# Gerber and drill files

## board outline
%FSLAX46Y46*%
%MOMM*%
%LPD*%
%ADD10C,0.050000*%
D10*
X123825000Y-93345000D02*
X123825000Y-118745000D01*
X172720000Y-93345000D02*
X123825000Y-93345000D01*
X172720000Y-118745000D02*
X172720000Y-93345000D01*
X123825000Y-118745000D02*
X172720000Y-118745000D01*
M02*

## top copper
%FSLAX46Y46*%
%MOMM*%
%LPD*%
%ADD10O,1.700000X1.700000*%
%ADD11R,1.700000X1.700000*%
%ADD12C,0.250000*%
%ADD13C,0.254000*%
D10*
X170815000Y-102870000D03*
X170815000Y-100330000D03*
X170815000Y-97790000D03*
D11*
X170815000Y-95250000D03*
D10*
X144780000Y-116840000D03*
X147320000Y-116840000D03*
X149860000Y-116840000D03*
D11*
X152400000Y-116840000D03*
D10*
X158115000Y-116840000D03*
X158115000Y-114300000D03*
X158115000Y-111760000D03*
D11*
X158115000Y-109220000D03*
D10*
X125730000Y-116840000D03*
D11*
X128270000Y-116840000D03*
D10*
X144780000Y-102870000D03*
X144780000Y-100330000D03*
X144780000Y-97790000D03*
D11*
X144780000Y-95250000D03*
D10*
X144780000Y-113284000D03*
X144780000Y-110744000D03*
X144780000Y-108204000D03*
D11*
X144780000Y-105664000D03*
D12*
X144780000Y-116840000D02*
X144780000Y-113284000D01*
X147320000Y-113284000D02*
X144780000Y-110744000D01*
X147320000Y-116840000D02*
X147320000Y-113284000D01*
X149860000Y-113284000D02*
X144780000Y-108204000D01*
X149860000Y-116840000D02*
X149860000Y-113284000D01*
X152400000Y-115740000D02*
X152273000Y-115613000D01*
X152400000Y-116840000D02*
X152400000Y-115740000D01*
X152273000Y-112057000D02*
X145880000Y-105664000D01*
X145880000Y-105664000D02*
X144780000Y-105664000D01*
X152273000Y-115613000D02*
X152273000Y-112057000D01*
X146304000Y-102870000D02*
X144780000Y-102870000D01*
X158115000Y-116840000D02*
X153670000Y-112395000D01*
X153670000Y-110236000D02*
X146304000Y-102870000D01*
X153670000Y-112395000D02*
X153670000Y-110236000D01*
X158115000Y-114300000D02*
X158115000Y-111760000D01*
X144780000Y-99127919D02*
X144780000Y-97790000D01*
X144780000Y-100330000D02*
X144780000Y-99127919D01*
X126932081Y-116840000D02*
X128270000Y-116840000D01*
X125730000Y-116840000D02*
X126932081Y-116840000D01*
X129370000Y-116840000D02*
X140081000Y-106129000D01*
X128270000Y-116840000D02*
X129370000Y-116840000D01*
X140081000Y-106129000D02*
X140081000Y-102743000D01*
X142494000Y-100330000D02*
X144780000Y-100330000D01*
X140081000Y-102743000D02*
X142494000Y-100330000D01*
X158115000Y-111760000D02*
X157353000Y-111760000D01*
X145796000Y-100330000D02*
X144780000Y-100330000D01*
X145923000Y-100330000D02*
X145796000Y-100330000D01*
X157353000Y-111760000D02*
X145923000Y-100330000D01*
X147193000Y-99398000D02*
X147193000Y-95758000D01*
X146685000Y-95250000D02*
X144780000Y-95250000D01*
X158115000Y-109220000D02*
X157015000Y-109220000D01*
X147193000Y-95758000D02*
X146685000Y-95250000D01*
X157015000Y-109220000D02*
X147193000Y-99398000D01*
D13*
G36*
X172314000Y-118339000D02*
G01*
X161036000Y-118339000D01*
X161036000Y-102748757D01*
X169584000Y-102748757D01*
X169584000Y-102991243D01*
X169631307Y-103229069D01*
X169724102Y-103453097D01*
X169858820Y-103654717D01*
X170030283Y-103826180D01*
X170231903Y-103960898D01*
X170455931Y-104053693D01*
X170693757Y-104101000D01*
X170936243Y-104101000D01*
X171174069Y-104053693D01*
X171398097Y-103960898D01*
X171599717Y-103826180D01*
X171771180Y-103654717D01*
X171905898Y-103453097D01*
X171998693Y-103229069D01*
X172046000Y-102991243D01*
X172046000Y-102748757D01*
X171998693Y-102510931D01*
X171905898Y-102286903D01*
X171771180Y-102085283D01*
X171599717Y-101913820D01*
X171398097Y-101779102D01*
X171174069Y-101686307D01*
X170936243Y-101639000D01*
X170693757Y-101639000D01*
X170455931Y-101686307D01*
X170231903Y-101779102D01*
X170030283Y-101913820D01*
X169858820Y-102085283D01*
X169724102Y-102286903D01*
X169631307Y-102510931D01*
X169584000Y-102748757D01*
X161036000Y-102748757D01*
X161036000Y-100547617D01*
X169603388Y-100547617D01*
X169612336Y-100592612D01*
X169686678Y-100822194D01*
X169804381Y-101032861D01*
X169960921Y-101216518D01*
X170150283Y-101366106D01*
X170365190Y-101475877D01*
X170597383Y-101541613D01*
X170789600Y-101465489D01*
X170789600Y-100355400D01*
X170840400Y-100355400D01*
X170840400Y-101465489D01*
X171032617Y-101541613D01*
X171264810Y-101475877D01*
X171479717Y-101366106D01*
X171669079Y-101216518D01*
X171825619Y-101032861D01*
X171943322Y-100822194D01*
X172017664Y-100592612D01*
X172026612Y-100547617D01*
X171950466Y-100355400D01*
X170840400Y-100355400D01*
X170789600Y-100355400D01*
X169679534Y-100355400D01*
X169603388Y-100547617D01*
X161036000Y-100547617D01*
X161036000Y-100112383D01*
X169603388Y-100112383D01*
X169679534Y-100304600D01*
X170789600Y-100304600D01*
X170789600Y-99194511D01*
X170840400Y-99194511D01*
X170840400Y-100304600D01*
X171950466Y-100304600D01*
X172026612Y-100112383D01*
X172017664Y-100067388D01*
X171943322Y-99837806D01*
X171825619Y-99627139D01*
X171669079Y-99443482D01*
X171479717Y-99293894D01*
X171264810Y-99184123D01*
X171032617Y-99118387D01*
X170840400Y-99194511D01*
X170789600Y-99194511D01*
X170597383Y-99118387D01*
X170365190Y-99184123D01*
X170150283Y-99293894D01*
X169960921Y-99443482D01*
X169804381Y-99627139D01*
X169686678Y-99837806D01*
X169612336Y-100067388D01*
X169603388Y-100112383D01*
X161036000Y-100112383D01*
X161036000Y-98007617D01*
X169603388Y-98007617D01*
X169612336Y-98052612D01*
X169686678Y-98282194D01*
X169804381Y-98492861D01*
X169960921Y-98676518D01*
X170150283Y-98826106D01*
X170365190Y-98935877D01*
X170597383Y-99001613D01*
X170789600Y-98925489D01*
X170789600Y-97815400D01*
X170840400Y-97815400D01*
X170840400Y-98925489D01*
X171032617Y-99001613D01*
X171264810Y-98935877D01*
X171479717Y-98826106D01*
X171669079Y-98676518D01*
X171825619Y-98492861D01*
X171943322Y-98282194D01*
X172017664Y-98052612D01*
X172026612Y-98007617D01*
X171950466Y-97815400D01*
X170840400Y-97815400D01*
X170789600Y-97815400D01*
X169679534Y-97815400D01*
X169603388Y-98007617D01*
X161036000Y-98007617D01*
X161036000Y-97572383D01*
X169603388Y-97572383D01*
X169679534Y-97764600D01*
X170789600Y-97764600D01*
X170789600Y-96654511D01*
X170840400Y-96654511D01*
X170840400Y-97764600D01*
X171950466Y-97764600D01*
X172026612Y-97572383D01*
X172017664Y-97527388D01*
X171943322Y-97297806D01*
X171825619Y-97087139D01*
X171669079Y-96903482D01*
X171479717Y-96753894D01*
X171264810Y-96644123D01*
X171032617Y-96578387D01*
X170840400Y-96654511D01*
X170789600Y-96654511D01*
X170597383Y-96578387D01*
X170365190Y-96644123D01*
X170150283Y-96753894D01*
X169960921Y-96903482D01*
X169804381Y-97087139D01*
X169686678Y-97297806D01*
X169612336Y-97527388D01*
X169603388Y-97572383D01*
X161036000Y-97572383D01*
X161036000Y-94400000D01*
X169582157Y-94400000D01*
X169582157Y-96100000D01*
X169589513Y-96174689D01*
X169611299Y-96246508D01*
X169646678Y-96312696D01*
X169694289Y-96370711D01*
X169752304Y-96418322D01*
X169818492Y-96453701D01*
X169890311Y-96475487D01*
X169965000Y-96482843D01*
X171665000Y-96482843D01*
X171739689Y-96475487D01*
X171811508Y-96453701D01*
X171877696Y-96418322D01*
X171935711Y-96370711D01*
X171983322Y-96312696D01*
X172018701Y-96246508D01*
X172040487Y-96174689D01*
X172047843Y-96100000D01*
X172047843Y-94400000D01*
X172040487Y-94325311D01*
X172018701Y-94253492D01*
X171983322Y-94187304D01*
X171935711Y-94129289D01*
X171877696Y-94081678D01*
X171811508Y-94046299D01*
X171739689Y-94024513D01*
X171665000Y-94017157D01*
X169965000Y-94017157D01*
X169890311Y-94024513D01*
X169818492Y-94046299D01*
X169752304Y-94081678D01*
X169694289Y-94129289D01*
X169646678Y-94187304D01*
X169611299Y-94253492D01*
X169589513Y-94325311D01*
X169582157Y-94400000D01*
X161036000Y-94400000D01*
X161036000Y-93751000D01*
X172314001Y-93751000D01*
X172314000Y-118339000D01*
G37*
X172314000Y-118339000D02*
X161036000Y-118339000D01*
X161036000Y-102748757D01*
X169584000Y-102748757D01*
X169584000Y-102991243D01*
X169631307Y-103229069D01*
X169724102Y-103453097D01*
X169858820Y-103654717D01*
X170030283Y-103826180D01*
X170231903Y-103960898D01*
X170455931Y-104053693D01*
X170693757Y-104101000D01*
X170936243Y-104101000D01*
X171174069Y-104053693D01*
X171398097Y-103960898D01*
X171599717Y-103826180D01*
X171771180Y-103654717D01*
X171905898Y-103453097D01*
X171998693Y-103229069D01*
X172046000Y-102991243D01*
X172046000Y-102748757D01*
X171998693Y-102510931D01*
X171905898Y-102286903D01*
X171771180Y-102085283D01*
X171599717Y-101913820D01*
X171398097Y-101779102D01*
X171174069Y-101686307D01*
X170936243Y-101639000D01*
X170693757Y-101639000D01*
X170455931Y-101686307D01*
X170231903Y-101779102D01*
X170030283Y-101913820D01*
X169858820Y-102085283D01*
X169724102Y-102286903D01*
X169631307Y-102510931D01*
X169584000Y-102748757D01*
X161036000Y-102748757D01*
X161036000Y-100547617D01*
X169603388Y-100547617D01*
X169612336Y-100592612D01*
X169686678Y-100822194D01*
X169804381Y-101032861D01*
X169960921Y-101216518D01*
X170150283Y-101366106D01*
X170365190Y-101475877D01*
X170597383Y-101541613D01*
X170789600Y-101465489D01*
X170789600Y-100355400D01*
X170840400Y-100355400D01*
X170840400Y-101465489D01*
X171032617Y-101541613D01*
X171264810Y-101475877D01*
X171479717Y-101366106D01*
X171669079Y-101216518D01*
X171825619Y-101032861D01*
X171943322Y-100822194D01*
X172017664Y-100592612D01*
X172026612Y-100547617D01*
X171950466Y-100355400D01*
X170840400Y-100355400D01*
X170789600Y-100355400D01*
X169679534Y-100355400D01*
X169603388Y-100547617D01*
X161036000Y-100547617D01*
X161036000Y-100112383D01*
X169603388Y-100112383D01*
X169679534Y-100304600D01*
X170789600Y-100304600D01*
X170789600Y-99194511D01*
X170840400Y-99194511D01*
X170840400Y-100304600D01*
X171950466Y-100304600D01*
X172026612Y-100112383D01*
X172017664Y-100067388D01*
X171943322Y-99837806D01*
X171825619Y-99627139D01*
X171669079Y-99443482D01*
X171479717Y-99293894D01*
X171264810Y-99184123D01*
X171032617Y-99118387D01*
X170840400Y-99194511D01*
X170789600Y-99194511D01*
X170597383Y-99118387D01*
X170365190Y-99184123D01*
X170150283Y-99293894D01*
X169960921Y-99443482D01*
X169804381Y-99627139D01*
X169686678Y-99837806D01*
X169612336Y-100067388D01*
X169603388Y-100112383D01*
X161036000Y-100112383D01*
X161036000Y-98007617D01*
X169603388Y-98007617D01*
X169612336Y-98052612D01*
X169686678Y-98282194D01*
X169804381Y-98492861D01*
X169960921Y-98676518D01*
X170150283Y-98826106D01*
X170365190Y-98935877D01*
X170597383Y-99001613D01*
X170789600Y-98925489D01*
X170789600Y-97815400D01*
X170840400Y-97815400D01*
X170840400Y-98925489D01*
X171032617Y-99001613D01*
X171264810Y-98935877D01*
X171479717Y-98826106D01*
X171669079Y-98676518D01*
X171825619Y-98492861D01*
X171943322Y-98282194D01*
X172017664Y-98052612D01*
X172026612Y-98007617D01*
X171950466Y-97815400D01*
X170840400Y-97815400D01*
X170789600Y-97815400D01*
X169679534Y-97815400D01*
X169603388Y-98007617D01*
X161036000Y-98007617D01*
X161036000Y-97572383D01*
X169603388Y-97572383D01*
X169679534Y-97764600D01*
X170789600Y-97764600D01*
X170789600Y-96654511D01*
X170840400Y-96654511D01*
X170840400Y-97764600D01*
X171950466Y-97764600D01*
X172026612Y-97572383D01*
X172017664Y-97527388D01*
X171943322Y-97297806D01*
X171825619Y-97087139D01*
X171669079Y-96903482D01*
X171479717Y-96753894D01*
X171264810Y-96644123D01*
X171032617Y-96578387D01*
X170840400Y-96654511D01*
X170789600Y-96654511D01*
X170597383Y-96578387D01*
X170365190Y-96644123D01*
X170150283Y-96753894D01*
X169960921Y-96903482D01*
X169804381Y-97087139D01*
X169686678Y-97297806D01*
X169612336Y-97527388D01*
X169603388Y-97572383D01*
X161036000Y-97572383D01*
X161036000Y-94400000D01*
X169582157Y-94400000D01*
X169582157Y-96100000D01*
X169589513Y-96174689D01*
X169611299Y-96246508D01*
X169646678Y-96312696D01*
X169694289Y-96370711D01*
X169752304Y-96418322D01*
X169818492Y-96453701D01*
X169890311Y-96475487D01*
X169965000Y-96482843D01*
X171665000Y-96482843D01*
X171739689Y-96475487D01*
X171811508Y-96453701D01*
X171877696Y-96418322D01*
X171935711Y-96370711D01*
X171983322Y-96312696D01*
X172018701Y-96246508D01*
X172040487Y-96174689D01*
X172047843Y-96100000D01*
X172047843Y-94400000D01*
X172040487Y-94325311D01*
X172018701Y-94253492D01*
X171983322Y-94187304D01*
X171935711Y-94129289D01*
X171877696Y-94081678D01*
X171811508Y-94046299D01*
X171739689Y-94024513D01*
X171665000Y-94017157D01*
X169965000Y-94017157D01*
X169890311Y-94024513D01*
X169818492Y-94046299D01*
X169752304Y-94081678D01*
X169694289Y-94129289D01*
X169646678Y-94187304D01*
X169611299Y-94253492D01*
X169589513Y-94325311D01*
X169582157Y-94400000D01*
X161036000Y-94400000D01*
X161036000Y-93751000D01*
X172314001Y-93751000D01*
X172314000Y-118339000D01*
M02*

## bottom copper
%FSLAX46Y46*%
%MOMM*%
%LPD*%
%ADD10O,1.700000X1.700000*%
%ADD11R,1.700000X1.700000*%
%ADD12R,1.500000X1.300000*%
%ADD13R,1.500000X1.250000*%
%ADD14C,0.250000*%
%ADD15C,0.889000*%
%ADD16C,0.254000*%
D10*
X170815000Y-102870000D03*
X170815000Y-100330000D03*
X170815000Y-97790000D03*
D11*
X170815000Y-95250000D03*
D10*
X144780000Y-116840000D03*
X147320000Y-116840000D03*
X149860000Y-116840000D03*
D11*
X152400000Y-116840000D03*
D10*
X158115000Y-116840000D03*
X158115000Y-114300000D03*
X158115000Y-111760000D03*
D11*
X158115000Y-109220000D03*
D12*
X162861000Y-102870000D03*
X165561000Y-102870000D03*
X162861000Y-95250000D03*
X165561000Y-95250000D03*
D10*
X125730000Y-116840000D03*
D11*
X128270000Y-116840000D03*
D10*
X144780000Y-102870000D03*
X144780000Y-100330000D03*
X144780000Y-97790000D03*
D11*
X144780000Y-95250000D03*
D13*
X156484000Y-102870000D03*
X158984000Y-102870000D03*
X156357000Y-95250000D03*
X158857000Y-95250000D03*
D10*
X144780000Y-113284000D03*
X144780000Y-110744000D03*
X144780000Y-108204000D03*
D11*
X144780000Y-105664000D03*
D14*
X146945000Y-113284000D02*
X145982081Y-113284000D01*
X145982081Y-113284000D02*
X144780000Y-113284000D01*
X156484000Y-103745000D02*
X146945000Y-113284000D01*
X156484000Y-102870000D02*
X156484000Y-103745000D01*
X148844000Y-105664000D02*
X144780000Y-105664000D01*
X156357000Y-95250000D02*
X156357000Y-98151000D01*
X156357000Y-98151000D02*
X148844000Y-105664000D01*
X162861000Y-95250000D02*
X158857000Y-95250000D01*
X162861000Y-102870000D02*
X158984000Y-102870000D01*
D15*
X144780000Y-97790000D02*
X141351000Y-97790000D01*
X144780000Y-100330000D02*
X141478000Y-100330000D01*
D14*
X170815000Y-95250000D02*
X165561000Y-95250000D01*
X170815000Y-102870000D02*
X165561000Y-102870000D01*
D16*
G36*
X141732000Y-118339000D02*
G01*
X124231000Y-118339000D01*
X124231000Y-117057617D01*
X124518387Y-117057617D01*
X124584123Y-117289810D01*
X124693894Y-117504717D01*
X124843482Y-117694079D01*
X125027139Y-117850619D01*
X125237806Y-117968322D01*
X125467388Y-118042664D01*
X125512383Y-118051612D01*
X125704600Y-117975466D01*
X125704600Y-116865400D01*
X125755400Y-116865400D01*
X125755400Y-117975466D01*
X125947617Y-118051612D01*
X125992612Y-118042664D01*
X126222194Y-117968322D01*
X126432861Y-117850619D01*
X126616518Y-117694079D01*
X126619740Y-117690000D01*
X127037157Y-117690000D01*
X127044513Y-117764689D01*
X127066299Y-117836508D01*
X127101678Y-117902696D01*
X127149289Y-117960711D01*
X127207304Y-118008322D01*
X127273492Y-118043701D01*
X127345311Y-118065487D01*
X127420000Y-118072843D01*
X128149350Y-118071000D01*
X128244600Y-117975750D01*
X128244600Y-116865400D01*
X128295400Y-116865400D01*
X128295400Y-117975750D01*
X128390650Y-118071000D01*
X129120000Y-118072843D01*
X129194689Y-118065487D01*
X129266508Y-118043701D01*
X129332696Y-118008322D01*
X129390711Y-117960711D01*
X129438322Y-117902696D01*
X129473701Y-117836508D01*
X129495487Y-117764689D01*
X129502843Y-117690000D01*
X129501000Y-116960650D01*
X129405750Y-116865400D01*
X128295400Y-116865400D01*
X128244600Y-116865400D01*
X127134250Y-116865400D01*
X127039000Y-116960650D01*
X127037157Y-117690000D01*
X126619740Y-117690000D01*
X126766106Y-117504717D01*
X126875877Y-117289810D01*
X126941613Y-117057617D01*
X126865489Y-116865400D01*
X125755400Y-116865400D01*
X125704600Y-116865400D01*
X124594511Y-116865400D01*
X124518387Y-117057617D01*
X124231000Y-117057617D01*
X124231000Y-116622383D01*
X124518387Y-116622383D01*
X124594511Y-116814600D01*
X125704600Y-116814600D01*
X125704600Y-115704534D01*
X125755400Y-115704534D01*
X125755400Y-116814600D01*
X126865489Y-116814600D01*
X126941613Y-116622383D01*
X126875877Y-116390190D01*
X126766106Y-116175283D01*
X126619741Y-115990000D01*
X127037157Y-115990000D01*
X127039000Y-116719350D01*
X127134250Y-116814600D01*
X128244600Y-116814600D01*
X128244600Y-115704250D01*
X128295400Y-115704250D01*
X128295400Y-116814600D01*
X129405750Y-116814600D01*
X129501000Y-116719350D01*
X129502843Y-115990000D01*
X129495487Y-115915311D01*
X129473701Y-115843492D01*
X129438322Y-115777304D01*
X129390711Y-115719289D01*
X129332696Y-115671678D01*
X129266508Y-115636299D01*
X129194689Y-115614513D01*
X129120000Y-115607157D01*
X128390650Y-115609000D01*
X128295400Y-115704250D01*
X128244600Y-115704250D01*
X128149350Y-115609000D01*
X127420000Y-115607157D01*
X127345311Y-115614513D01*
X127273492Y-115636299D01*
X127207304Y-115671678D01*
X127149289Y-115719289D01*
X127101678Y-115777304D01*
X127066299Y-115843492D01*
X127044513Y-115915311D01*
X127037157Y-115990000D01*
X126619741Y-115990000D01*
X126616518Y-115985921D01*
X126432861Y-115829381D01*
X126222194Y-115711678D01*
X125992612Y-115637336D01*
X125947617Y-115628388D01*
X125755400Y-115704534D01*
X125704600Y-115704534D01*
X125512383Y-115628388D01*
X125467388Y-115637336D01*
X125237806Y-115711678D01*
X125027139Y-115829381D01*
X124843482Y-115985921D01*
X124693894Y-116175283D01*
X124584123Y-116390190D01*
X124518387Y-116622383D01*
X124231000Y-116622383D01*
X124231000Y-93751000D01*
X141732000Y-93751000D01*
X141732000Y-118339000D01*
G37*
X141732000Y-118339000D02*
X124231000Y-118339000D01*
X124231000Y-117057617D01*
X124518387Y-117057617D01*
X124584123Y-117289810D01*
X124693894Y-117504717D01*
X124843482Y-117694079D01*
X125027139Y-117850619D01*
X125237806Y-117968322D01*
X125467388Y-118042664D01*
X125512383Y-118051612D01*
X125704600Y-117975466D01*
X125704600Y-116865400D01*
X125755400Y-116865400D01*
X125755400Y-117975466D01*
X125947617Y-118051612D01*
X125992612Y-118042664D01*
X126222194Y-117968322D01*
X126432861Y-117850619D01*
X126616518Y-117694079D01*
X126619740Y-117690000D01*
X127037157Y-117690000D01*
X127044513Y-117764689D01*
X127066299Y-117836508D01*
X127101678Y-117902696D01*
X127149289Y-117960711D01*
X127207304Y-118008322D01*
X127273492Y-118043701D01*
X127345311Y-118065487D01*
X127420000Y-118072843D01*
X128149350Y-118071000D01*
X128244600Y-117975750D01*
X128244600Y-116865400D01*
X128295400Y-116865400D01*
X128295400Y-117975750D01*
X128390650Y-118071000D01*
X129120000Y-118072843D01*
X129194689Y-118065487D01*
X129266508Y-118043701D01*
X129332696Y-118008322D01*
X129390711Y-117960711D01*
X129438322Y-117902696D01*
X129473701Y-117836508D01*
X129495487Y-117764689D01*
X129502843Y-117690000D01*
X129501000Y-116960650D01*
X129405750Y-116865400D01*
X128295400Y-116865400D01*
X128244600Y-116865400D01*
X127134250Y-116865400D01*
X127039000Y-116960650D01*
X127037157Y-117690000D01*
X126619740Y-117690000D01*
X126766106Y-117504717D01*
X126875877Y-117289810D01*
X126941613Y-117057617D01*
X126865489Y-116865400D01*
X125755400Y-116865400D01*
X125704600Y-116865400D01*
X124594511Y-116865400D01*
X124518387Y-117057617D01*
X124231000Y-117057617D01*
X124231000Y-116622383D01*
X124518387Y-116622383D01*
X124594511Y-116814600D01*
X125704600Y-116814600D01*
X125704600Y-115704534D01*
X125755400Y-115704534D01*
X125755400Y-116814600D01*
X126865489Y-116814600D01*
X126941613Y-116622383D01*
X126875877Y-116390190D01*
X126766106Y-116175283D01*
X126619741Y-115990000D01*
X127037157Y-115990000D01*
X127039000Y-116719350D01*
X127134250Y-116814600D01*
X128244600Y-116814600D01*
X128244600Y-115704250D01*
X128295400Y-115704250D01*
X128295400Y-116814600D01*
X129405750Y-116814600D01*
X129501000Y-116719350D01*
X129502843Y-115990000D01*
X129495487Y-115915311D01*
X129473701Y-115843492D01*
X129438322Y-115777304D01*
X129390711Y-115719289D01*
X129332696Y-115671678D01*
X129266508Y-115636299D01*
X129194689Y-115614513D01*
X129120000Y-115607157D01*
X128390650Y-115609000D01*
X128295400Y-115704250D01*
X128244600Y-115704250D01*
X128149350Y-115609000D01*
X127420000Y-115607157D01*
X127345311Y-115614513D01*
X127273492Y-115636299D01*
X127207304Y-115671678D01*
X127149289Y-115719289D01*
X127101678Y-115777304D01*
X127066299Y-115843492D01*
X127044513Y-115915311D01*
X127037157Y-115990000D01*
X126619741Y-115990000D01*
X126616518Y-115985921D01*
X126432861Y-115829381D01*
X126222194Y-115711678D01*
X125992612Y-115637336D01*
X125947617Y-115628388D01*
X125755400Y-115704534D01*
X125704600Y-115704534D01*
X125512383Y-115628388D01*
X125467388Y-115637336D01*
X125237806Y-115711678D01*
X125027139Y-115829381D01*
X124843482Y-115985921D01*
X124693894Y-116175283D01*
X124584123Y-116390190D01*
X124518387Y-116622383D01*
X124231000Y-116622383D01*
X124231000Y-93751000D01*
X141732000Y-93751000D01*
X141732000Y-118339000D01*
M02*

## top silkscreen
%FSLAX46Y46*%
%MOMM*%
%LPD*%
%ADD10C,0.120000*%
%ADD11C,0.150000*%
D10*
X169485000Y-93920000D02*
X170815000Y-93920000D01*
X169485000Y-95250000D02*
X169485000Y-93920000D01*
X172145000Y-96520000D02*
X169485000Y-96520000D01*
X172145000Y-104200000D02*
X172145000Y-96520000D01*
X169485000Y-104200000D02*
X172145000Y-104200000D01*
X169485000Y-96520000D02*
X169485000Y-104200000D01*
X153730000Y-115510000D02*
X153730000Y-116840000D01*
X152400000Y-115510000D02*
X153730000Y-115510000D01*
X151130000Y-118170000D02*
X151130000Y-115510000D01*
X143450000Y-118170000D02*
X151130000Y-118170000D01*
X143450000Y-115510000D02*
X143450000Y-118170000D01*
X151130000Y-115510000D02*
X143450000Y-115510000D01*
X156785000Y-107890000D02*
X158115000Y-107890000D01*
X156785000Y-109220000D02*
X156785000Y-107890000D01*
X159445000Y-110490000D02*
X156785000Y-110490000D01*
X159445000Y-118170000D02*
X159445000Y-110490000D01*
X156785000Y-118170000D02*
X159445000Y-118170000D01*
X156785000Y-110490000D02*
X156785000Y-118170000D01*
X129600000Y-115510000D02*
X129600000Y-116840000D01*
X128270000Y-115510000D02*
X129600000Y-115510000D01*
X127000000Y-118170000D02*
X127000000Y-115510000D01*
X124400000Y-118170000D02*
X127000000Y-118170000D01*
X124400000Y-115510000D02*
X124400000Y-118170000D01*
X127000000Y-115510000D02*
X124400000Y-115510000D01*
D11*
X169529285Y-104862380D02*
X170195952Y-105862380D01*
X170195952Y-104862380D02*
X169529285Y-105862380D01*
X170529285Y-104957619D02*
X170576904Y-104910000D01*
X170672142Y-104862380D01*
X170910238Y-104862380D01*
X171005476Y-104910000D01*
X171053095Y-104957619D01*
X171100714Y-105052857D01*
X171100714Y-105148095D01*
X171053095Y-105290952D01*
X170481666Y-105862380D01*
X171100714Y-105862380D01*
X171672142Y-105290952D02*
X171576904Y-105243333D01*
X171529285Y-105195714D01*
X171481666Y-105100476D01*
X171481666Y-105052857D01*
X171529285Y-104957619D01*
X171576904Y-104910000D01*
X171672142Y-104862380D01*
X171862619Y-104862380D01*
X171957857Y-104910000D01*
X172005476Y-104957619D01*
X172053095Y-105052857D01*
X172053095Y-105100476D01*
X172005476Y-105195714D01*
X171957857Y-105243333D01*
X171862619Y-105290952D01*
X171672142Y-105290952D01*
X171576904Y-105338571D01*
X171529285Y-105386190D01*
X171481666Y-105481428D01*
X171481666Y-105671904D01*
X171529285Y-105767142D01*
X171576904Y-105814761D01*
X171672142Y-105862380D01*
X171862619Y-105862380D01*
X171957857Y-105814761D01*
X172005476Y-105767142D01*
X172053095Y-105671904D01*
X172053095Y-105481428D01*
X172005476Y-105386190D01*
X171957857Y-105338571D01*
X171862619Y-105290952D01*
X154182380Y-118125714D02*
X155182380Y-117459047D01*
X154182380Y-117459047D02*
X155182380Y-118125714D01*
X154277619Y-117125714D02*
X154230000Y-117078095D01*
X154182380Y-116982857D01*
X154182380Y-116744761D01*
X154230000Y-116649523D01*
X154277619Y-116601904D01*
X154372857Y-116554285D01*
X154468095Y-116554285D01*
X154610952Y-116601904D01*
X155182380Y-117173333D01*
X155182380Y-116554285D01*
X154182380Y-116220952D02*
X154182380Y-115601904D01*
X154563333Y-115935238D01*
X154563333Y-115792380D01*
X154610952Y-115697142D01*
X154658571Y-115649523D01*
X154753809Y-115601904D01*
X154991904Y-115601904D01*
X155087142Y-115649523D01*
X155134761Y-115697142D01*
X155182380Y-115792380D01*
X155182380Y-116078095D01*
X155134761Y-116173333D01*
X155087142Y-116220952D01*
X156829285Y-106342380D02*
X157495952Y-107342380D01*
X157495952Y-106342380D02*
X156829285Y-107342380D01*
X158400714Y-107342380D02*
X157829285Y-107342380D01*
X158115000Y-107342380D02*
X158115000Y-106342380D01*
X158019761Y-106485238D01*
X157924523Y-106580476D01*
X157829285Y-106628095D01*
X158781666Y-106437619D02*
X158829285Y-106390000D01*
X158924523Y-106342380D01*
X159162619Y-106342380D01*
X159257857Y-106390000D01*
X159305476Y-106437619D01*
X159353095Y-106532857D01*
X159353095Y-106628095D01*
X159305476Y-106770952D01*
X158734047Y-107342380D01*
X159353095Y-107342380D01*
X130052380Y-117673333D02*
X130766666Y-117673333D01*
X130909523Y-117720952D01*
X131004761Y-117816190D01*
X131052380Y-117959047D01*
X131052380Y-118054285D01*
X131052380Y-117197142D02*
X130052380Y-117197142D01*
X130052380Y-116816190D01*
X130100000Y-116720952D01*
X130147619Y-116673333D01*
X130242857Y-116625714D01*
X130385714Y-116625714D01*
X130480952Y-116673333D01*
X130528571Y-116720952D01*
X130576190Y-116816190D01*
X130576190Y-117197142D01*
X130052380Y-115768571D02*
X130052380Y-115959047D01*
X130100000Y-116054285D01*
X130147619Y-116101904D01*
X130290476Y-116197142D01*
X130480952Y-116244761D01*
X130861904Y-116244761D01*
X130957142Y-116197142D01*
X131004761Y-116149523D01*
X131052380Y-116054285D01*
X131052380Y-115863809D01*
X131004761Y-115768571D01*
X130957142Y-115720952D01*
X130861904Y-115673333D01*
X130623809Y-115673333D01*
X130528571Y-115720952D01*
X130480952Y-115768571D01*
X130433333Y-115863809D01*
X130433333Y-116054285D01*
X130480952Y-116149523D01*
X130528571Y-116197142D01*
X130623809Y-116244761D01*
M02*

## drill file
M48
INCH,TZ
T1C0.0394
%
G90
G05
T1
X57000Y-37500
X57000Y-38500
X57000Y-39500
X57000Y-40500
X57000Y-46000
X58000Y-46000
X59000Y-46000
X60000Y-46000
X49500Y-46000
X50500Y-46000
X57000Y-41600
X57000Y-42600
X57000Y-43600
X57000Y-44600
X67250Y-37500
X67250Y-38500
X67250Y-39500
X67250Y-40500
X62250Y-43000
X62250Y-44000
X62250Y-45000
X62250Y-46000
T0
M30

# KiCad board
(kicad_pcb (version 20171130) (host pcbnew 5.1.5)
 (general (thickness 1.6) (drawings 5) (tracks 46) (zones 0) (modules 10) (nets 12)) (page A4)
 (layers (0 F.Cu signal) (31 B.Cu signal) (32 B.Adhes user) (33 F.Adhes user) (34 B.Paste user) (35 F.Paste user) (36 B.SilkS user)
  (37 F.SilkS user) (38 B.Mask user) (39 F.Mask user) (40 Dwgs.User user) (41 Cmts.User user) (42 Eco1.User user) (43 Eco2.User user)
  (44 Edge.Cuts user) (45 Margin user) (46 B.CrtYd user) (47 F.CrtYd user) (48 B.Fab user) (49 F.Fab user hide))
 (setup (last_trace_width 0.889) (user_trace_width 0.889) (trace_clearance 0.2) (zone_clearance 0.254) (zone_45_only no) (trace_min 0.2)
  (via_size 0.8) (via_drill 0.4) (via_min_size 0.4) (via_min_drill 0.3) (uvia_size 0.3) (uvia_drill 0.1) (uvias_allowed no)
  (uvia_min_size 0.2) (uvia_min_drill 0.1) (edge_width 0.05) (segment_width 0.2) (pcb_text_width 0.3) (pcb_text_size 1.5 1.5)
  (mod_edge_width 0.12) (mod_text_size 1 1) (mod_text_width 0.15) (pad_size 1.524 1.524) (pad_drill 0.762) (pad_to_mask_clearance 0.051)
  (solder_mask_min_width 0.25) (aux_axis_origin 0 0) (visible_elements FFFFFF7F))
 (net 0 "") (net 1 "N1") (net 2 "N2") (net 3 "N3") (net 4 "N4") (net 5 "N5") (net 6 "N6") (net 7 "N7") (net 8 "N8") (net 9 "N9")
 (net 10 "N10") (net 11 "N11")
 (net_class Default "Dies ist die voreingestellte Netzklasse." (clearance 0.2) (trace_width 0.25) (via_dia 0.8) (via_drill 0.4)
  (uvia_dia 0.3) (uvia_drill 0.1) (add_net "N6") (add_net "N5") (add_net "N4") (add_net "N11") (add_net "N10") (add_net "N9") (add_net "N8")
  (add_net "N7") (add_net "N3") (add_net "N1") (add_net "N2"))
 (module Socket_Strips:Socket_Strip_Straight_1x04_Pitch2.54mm (layer F.Cu) (at 170.815 95.25)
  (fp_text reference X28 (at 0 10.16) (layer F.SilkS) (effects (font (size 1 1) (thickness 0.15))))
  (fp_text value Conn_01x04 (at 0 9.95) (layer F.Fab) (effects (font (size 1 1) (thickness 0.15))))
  (fp_line (start -1.33 -1.33) (end 0 -1.33) (layer F.SilkS) (width 0.12))
  (fp_line (start -1.33 0) (end -1.33 -1.33) (layer F.SilkS) (width 0.12))
  (fp_line (start 1.33 1.27) (end -1.33 1.27) (layer F.SilkS) (width 0.12))
  (fp_line (start 1.33 8.95) (end 1.33 1.27) (layer F.SilkS) (width 0.12))
  (fp_line (start -1.33 8.95) (end 1.33 8.95) (layer F.SilkS) (width 0.12))
  (fp_line (start -1.33 1.27) (end -1.33 8.95) (layer F.SilkS) (width 0.12))
  (pad 4 thru_hole oval (at 0 7.62) (size 1.7 1.7) (drill 1) (layers *.Cu *.Mask) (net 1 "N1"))
  (pad 3 thru_hole oval (at 0 5.08) (size 1.7 1.7) (drill 1) (layers *.Cu *.Mask) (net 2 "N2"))
  (pad 2 thru_hole oval (at 0 2.54) (size 1.7 1.7) (drill 1) (layers *.Cu *.Mask) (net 2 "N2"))
  (pad 1 thru_hole rect (at 0 0) (size 1.7 1.7) (drill 1) (layers *.Cu *.Mask) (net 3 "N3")))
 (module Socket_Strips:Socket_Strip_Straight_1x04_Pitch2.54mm (layer F.Cu) (at 152.4 116.84 270)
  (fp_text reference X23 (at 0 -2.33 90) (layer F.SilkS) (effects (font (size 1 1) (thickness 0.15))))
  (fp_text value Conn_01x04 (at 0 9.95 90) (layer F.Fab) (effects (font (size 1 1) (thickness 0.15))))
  (fp_line (start -1.33 -1.33) (end 0 -1.33) (layer F.SilkS) (width 0.12))
  (fp_line (start -1.33 0) (end -1.33 -1.33) (layer F.SilkS) (width 0.12))
  (fp_line (start 1.33 1.27) (end -1.33 1.27) (layer F.SilkS) (width 0.12))
  (fp_line (start 1.33 8.95) (end 1.33 1.27) (layer F.SilkS) (width 0.12))
  (fp_line (start -1.33 8.95) (end 1.33 8.95) (layer F.SilkS) (width 0.12))
  (fp_line (start -1.33 1.27) (end -1.33 8.95) (layer F.SilkS) (width 0.12))
  (pad 4 thru_hole oval (at 0 7.62 270) (size 1.7 1.7) (drill 1) (layers *.Cu *.Mask) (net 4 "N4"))
  (pad 3 thru_hole oval (at 0 5.08 270) (size 1.7 1.7) (drill 1) (layers *.Cu *.Mask) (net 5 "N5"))
  (pad 2 thru_hole oval (at 0 2.54 270) (size 1.7 1.7) (drill 1) (layers *.Cu *.Mask) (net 5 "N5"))
  (pad 1 thru_hole rect (at 0 0 270) (size 1.7 1.7) (drill 1) (layers *.Cu *.Mask) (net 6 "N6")))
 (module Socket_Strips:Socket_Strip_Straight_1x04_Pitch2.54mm (layer F.Cu) (at 158.115 109.22)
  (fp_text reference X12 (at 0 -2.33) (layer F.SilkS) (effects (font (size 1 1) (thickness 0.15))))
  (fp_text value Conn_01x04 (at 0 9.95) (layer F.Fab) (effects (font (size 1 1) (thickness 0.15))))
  (fp_line (start -1.33 -1.33) (end 0 -1.33) (layer F.SilkS) (width 0.12))
  (fp_line (start -1.33 0) (end -1.33 -1.33) (layer F.SilkS) (width 0.12))
  (fp_line (start 1.33 1.27) (end -1.33 1.27) (layer F.SilkS) (width 0.12))
  (fp_line (start 1.33 8.95) (end 1.33 1.27) (layer F.SilkS) (width 0.12))
  (fp_line (start -1.33 8.95) (end 1.33 8.95) (layer F.SilkS) (width 0.12))
  (fp_line (start -1.33 1.27) (end -1.33 8.95) (layer F.SilkS) (width 0.12))
  (pad 4 thru_hole oval (at 0 7.62) (size 1.7 1.7) (drill 1) (layers *.Cu *.Mask) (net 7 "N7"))
  (pad 3 thru_hole oval (at 0 5.08) (size 1.7 1.7) (drill 1) (layers *.Cu *.Mask) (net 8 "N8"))
  (pad 2 thru_hole oval (at 0 2.54) (size 1.7 1.7) (drill 1) (layers *.Cu *.Mask) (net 8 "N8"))
  (pad 1 thru_hole rect (at 0 0) (size 1.7 1.7) (drill 1) (layers *.Cu *.Mask) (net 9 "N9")))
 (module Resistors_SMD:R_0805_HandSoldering (layer B.Cu) (at 164.211 102.87 180)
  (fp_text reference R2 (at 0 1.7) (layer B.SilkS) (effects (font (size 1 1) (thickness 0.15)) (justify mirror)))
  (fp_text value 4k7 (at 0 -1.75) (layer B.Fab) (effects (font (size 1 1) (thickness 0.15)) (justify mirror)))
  (pad 2 smd rect (at 1.35 0 180) (size 1.5 1.3) (layers B.Cu B.Paste B.Mask) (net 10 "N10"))
  (pad 1 smd rect (at -1.35 0 180) (size 1.5 1.3) (layers B.Cu B.Paste B.Mask) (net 1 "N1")))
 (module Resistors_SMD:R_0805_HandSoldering (layer B.Cu) (at 164.211 95.25 180)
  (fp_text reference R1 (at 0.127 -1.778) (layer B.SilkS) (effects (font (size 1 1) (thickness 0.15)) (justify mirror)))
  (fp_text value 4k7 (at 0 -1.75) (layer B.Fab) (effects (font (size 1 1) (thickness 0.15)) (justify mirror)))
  (pad 2 smd rect (at 1.35 0 180) (size 1.5 1.3) (layers B.Cu B.Paste B.Mask) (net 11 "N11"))
  (pad 1 smd rect (at -1.35 0 180) (size 1.5 1.3) (layers B.Cu B.Paste B.Mask) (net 3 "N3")))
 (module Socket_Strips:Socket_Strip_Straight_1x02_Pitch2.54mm (layer F.Cu) (at 128.27 116.84 270)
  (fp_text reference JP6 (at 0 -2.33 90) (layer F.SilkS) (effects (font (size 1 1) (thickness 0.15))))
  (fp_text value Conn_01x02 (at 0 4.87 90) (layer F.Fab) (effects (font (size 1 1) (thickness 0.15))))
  (fp_line (start -1.33 -1.33) (end 0 -1.33) (layer F.SilkS) (width 0.12))
  (fp_line (start -1.33 0) (end -1.33 -1.33) (layer F.SilkS) (width 0.12))
  (fp_line (start 1.33 1.27) (end -1.33 1.27) (layer F.SilkS) (width 0.12))
  (fp_line (start 1.33 3.87) (end 1.33 1.27) (layer F.SilkS) (width 0.12))
  (fp_line (start -1.33 3.87) (end 1.33 3.87) (layer F.SilkS) (width 0.12))
  (fp_line (start -1.33 1.27) (end -1.33 3.87) (layer F.SilkS) (width 0.12))
  (pad 2 thru_hole oval (at 0 2.54 270) (size 1.7 1.7) (drill 1) (layers *.Cu *.Mask) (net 8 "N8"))
  (pad 1 thru_hole rect (at 0 0 270) (size 1.7 1.7) (drill 1) (layers *.Cu *.Mask) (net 8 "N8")))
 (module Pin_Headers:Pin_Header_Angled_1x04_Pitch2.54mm (layer B.Cu) (at 144.78 95.25 180)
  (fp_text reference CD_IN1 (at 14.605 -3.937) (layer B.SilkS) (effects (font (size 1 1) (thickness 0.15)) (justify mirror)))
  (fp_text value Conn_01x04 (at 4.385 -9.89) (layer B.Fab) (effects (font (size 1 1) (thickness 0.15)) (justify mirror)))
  (pad 4 thru_hole oval (at 0 -7.62 180) (size 1.7 1.7) (drill 1) (layers *.Cu *.Mask) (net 7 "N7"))
  (pad 3 thru_hole oval (at 0 -5.08 180) (size 1.7 1.7) (drill 1) (layers *.Cu *.Mask) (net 8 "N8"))
  (pad 2 thru_hole oval (at 0 -2.54 180) (size 1.7 1.7) (drill 1) (layers *.Cu *.Mask) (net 8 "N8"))
  (pad 1 thru_hole rect (at 0 0 180) (size 1.7 1.7) (drill 1) (layers *.Cu *.Mask) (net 9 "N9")))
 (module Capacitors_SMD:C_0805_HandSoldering (layer B.Cu) (at 157.734 102.87 180)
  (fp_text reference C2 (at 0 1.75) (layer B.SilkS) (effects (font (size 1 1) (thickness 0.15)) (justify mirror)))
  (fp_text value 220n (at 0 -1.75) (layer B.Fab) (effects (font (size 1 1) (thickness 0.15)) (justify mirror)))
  (pad 2 smd rect (at 1.25 0 180) (size 1.5 1.25) (layers B.Cu B.Paste B.Mask) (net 4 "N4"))
  (pad 1 smd rect (at -1.25 0 180) (size 1.5 1.25) (layers B.Cu B.Paste B.Mask) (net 10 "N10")))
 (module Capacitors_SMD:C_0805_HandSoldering (layer B.Cu) (at 157.607 95.25 180)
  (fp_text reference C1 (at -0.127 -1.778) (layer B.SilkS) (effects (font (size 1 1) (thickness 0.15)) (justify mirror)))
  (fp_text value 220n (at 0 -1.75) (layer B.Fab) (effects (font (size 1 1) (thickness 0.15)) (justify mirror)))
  (pad 2 smd rect (at 1.25 0 180) (size 1.5 1.25) (layers B.Cu B.Paste B.Mask) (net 6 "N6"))
  (pad 1 smd rect (at -1.25 0 180) (size 1.5 1.25) (layers B.Cu B.Paste B.Mask) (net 11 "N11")))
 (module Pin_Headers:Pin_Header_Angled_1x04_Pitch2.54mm (layer B.Cu) (at 144.78 105.664 180)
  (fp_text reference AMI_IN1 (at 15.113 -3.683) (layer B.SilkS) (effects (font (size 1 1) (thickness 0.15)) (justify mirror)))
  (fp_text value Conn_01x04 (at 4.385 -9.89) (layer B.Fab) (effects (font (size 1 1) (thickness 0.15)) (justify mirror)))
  (pad 4 thru_hole oval (at 0 -7.62 180) (size 1.7 1.7) (drill 1) (layers *.Cu *.Mask) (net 4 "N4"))
  (pad 3 thru_hole oval (at 0 -5.08 180) (size 1.7 1.7) (drill 1) (layers *.Cu *.Mask) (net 5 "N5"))
  (pad 2 thru_hole oval (at 0 -2.54 180) (size 1.7 1.7) (drill 1) (layers *.Cu *.Mask) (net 5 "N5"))
  (pad 1 thru_hole rect (at 0 0 180) (size 1.7 1.7) (drill 1) (layers *.Cu *.Mask) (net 6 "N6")))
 (gr_line (start 123.825 93.345) (end 123.825 118.745) (layer Edge.Cuts) (width 0.05))
 (gr_line (start 172.72 93.345) (end 123.825 93.345) (layer Edge.Cuts) (width 0.05))
 (gr_line (start 172.72 118.745) (end 172.72 93.345) (layer Edge.Cuts) (width 0.05))
 (gr_line (start 123.825 118.745) (end 172.72 118.745) (layer Edge.Cuts) (width 0.05))
 (segment (start 144.78 116.84) (end 144.78 113.284) (width 0.25) (layer F.Cu) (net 4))
 (segment (start 146.945 113.284) (end 145.982081 113.284) (width 0.25) (layer B.Cu) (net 4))
 (segment (start 145.982081 113.284) (end 144.78 113.284) (width 0.25) (layer B.Cu) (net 4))
 (segment (start 156.484 103.745) (end 146.945 113.284) (width 0.25) (layer B.Cu) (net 4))
 (segment (start 156.484 102.87) (end 156.484 103.745) (width 0.25) (layer B.Cu) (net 4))
 (segment (start 147.32 113.284) (end 144.78 110.744) (width 0.25) (layer F.Cu) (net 5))
 (segment (start 147.32 116.84) (end 147.32 113.284) (width 0.25) (layer F.Cu) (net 5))
 (segment (start 149.86 113.284) (end 144.78 108.204) (width 0.25) (layer F.Cu) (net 5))
 (segment (start 149.86 116.84) (end 149.86 113.284) (width 0.25) (layer F.Cu) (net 5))
 (segment (start 152.4 115.74) (end 152.273 115.613) (width 0.25) (layer F.Cu) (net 6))
 (segment (start 152.4 116.84) (end 152.4 115.74) (width 0.25) (layer F.Cu) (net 6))
 (segment (start 152.273 112.057) (end 145.88 105.664) (width 0.25) (layer F.Cu) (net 6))
 (segment (start 145.88 105.664) (end 144.78 105.664) (width 0.25) (layer F.Cu) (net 6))
 (segment (start 152.273 115.613) (end 152.273 112.057) (width 0.25) (layer F.Cu) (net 6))
 (segment (start 148.844 105.664) (end 144.78 105.664) (width 0.25) (layer B.Cu) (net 6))
 (segment (start 156.357 95.25) (end 156.357 98.151) (width 0.25) (layer B.Cu) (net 6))
 (segment (start 156.357 98.151) (end 148.844 105.664) (width 0.25) (layer B.Cu) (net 6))
 (segment (start 162.861 95.25) (end 158.857 95.25) (width 0.25) (layer B.Cu) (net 11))
 (segment (start 162.861 102.87) (end 158.984 102.87) (width 0.25) (layer B.Cu) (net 10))
 (segment (start 146.304 102.87) (end 144.78 102.87) (width 0.25) (layer F.Cu) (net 7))
 (segment (start 158.115 116.84) (end 153.67 112.395) (width 0.25) (layer F.Cu) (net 7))
 (segment (start 153.67 110.236) (end 146.304 102.87) (width 0.25) (layer F.Cu) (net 7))
 (segment (start 153.67 112.395) (end 153.67 110.236) (width 0.25) (layer F.Cu) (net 7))
 (segment (start 158.115 114.3) (end 158.115 111.76) (width 0.25) (layer F.Cu) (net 8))
 (segment (start 144.78 99.127919) (end 144.78 97.79) (width 0.25) (layer F.Cu) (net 8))
 (segment (start 144.78 100.33) (end 144.78 99.127919) (width 0.25) (layer F.Cu) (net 8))
 (segment (start 126.932081 116.84) (end 128.27 116.84) (width 0.25) (layer F.Cu) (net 8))
 (segment (start 125.73 116.84) (end 126.932081 116.84) (width 0.25) (layer F.Cu) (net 8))
 (segment (start 129.37 116.84) (end 140.081 106.129) (width 0.25) (layer F.Cu) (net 8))
 (segment (start 128.27 116.84) (end 129.37 116.84) (width 0.25) (layer F.Cu) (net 8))
 (segment (start 140.081 106.129) (end 140.081 102.743) (width 0.25) (layer F.Cu) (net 8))
 (segment (start 142.494 100.33) (end 144.78 100.33) (width 0.25) (layer F.Cu) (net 8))
 (segment (start 140.081 102.743) (end 142.494 100.33) (width 0.25) (layer F.Cu) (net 8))
 (segment (start 158.115 111.76) (end 157.353 111.76) (width 0.25) (layer F.Cu) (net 8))
 (segment (start 145.796 100.33) (end 144.78 100.33) (width 0.25) (layer F.Cu) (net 8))
 (segment (start 145.923 100.33) (end 145.796 100.33) (width 0.25) (layer F.Cu) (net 8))
 (segment (start 157.353 111.76) (end 145.923 100.33) (width 0.25) (layer F.Cu) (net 8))
 (segment (start 144.78 97.79) (end 141.351 97.79) (width 0.889) (layer B.Cu) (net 8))
 (segment (start 144.78 100.33) (end 141.478 100.33) (width 0.889) (layer B.Cu) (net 8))
 (segment (start 147.193 99.398) (end 147.193 95.758) (width 0.25) (layer F.Cu) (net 9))
 (segment (start 146.685 95.25) (end 144.78 95.25) (width 0.25) (layer F.Cu) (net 9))
 (segment (start 158.115 109.22) (end 157.015 109.22) (width 0.25) (layer F.Cu) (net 9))
 (segment (start 147.193 95.758) (end 146.685 95.25) (width 0.25) (layer F.Cu) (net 9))
 (segment (start 157.015 109.22) (end 147.193 99.398) (width 0.25) (layer F.Cu) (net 9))
 (segment (start 170.815 95.25) (end 165.561 95.25) (width 0.25) (layer B.Cu) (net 3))
 (segment (start 170.815 102.87) (end 165.561 102.87) (width 0.25) (layer B.Cu) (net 1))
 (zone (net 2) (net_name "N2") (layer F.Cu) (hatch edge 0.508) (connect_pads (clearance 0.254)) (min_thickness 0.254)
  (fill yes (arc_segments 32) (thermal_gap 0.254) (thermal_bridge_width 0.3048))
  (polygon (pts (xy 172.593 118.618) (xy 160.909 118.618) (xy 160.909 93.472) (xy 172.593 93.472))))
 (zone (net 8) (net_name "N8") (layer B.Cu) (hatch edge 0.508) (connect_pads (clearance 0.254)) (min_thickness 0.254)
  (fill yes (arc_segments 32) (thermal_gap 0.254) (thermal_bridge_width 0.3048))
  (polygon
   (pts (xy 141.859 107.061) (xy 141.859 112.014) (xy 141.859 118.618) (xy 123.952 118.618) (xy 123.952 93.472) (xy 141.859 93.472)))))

